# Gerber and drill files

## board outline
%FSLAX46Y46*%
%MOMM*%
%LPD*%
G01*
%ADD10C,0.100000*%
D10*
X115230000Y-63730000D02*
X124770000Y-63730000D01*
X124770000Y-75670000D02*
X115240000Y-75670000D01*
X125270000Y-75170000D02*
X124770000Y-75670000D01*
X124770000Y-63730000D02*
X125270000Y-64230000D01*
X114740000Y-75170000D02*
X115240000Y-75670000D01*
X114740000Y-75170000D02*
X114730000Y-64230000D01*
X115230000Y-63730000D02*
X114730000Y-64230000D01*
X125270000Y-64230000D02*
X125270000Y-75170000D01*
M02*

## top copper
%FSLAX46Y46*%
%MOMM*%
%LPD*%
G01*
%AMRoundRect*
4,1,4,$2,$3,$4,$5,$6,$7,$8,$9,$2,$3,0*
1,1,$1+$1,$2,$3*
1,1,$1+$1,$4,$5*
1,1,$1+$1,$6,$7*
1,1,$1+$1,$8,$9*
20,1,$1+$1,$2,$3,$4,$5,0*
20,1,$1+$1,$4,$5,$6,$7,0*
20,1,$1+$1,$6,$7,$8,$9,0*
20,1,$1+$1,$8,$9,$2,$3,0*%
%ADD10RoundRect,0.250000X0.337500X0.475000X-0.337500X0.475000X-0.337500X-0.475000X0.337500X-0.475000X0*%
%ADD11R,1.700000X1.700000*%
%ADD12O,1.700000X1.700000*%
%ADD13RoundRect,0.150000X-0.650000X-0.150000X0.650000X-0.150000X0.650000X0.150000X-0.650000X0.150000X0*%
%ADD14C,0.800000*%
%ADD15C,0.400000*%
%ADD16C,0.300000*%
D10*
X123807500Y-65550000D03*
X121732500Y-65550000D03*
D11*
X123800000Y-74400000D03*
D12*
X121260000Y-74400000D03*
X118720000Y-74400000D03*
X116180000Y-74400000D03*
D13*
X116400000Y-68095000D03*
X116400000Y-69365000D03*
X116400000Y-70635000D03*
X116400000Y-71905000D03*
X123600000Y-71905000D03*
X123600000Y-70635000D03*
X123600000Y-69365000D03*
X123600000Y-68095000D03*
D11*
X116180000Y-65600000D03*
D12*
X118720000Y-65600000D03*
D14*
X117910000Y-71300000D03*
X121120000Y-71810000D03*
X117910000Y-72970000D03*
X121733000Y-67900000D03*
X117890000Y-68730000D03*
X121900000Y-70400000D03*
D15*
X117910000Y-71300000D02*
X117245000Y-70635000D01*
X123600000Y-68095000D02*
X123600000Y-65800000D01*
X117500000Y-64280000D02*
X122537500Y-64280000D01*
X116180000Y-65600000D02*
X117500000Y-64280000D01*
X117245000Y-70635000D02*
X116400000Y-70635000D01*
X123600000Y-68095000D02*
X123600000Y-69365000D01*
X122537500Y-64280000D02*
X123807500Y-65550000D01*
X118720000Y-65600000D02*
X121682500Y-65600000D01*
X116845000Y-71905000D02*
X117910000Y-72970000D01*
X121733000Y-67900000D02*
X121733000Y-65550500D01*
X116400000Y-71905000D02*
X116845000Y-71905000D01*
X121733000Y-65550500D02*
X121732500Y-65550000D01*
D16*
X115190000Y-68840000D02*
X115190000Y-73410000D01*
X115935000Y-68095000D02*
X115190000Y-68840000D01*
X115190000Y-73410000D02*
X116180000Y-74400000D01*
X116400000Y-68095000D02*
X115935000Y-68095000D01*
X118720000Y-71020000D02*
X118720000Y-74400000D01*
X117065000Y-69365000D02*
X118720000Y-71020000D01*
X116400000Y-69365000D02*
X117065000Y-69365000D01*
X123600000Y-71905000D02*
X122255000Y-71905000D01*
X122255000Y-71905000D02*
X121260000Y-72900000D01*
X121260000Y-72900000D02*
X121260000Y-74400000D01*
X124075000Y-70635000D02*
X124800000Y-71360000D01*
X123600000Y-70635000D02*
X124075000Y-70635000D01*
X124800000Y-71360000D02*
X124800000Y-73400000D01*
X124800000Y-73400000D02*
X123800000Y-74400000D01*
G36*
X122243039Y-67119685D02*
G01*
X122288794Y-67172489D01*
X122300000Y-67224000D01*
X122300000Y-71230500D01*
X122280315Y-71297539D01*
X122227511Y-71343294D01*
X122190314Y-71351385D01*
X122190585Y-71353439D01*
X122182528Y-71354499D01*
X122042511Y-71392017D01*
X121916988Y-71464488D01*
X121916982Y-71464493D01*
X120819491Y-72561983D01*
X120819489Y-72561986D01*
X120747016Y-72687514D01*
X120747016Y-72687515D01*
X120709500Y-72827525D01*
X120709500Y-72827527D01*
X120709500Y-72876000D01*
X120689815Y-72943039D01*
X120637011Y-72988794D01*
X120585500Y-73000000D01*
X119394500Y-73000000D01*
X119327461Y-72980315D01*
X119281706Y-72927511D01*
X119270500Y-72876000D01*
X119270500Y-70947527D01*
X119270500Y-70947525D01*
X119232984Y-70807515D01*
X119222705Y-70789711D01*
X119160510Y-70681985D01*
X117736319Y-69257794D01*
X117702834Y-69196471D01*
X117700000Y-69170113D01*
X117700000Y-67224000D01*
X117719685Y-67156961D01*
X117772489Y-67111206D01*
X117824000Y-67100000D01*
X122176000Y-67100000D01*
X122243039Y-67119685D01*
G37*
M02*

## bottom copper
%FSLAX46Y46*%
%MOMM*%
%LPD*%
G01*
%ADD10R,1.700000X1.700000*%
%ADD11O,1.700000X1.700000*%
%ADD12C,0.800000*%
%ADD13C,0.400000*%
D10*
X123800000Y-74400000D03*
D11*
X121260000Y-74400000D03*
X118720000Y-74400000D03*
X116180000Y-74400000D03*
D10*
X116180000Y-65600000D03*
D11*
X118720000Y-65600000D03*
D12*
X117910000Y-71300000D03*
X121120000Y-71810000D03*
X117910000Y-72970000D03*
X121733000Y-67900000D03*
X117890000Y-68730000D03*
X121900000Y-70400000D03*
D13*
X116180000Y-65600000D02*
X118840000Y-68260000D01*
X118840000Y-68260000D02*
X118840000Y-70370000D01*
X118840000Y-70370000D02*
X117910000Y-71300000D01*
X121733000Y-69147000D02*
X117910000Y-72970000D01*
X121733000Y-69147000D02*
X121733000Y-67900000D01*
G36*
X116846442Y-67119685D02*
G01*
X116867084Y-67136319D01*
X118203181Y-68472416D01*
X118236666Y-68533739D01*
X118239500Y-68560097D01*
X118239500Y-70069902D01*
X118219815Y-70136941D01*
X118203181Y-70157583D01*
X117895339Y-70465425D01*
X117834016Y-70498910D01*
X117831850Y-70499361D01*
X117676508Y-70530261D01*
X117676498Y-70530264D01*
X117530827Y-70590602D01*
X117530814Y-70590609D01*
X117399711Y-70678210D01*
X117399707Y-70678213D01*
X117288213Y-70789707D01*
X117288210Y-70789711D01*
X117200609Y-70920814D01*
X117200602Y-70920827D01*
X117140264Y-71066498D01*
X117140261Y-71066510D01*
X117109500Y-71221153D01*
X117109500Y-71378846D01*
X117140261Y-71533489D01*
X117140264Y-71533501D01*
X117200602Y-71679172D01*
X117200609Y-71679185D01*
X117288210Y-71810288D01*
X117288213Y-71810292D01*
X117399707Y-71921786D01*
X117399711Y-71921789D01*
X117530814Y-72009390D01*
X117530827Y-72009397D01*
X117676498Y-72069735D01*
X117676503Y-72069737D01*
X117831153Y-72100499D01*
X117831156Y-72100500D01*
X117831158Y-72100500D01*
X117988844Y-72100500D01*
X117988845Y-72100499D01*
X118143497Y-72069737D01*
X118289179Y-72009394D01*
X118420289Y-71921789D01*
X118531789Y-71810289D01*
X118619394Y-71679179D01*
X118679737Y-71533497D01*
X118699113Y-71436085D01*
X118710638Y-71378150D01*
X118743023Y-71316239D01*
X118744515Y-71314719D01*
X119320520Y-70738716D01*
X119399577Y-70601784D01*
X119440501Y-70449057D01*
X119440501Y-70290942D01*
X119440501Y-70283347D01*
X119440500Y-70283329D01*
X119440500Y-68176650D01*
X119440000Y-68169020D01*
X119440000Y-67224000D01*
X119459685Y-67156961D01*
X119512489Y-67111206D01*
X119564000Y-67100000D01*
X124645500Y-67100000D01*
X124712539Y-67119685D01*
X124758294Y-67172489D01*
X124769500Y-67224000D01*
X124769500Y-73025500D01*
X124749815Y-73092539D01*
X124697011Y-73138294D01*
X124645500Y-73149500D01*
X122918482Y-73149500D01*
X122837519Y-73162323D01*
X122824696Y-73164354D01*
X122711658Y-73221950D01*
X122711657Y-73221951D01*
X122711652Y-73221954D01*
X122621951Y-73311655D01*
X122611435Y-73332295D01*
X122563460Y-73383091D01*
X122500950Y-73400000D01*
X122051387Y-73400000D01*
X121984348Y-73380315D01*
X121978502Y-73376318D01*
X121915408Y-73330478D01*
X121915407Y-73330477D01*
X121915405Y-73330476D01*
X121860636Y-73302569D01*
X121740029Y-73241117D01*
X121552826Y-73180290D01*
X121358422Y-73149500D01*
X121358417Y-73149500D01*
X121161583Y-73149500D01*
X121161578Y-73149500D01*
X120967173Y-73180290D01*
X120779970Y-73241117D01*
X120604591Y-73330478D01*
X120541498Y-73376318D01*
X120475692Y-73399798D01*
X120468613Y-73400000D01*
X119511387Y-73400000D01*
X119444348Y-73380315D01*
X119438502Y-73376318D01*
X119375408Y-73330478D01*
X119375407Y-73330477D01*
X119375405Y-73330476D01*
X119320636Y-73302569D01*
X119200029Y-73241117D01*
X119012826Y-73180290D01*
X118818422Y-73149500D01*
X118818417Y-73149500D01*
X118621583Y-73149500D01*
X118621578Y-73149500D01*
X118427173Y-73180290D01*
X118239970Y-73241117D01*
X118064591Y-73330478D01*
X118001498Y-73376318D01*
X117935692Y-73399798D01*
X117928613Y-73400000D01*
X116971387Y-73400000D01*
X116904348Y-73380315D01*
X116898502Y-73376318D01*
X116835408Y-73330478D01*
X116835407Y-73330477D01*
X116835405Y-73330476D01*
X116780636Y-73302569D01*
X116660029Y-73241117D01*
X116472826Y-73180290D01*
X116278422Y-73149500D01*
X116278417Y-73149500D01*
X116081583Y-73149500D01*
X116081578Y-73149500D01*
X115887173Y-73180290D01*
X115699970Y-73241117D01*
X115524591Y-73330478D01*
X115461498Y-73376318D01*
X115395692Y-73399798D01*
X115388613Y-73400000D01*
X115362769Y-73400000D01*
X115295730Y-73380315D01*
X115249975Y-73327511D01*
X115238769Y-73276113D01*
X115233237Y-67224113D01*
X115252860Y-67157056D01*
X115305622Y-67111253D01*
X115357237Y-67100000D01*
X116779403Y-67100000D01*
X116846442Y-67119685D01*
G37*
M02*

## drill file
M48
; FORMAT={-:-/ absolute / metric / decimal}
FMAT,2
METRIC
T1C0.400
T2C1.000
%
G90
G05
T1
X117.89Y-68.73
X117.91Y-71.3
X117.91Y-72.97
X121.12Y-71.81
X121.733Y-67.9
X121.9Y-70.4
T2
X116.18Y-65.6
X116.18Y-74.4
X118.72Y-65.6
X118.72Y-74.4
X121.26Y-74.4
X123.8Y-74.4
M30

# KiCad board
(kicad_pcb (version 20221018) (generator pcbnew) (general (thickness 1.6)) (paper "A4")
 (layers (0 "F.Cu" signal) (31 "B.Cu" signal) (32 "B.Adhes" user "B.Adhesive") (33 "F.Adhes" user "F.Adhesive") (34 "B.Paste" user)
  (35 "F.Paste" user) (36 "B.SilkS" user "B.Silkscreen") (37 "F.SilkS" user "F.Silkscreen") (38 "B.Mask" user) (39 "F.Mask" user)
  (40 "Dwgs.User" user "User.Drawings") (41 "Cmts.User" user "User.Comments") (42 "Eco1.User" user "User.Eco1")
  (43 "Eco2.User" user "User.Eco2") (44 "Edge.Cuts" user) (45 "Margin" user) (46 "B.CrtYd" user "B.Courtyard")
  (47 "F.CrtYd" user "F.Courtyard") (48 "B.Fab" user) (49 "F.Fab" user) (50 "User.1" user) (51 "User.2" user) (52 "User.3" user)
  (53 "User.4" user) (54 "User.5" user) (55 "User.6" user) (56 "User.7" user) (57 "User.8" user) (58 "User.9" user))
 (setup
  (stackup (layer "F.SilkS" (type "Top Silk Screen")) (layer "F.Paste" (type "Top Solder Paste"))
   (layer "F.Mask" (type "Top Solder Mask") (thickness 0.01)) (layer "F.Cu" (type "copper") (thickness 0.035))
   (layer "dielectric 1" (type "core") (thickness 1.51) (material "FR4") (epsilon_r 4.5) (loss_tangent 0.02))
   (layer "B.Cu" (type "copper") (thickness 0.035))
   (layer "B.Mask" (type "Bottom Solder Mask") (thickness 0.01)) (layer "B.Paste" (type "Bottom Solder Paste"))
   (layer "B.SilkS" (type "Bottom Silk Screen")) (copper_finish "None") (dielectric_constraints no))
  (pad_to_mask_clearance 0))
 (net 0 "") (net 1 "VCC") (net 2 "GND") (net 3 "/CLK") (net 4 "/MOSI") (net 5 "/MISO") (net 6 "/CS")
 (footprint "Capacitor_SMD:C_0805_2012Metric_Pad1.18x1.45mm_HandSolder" (layer "F.Cu") (at 122.77 65.55 180)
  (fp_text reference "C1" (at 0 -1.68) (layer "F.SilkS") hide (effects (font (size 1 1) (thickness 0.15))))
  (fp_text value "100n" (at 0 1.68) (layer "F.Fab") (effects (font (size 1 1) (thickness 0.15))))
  (pad "1" smd roundrect (at -1.0375 0 180) (size 1.175 1.45) (layers "F.Cu" "F.Paste" "F.Mask") (roundrect_rratio 0.2127659574)
   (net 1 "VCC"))
  (pad "2" smd roundrect (at 1.0375 0 180) (size 1.175 1.45) (layers "F.Cu" "F.Paste" "F.Mask") (roundrect_rratio 0.2127659574)
   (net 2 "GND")))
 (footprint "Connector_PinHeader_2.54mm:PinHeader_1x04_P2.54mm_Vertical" (layer "F.Cu") (at 123.8 74.4 -90)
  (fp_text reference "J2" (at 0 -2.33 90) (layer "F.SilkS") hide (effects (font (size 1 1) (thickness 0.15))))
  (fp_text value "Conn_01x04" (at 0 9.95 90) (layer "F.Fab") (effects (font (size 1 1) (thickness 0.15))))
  (pad "1" thru_hole rect (at 0 0 270) (size 1.7 1.7) (drill 1) (layers "*.Cu" "*.Mask") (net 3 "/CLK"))
  (pad "2" thru_hole oval (at 0 2.54 270) (size 1.7 1.7) (drill 1) (layers "*.Cu" "*.Mask") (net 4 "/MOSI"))
  (pad "3" thru_hole oval (at 0 5.08 270) (size 1.7 1.7) (drill 1) (layers "*.Cu" "*.Mask") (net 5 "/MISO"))
  (pad "4" thru_hole oval (at 0 7.62 270) (size 1.7 1.7) (drill 1) (layers "*.Cu" "*.Mask") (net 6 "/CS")))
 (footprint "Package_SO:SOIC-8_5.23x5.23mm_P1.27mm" (layer "F.Cu") (at 120 70)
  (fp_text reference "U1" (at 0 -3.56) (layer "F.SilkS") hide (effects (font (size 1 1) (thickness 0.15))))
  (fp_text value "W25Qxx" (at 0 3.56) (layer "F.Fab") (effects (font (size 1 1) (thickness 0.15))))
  (pad "1" smd roundrect (at -3.6 -1.905) (size 1.6 0.6) (layers "F.Cu" "F.Paste" "F.Mask") (roundrect_rratio 0.25) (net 6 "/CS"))
  (pad "2" smd roundrect (at -3.6 -0.635) (size 1.6 0.6) (layers "F.Cu" "F.Paste" "F.Mask") (roundrect_rratio 0.25) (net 5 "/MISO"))
  (pad "3" smd roundrect (at -3.6 0.635) (size 1.6 0.6) (layers "F.Cu" "F.Paste" "F.Mask") (roundrect_rratio 0.25) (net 1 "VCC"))
  (pad "4" smd roundrect (at -3.6 1.905) (size 1.6 0.6) (layers "F.Cu" "F.Paste" "F.Mask") (roundrect_rratio 0.25) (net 2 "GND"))
  (pad "5" smd roundrect (at 3.6 1.905) (size 1.6 0.6) (layers "F.Cu" "F.Paste" "F.Mask") (roundrect_rratio 0.25) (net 4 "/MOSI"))
  (pad "6" smd roundrect (at 3.6 0.635) (size 1.6 0.6) (layers "F.Cu" "F.Paste" "F.Mask") (roundrect_rratio 0.25) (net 3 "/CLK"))
  (pad "7" smd roundrect (at 3.6 -0.635) (size 1.6 0.6) (layers "F.Cu" "F.Paste" "F.Mask") (roundrect_rratio 0.25) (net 1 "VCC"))
  (pad "8" smd roundrect (at 3.6 -1.905) (size 1.6 0.6) (layers "F.Cu" "F.Paste" "F.Mask") (roundrect_rratio 0.25) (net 1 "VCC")))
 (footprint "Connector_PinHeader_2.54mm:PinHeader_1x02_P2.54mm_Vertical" (layer "F.Cu") (at 116.18 65.6 90)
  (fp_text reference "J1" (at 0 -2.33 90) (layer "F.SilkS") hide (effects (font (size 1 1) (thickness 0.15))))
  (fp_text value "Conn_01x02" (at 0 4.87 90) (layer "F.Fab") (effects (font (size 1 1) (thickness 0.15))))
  (pad "1" thru_hole rect (at 0 0 90) (size 1.7 1.7) (drill 1) (layers "*.Cu" "*.Mask") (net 1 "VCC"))
  (pad "2" thru_hole oval (at 0 2.54 90) (size 1.7 1.7) (drill 1) (layers "*.Cu" "*.Mask") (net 2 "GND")))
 (gr_line (start 115.23 63.73) (end 124.77 63.73) (stroke (width 0.1) (type default)) (layer "Edge.Cuts"))
 (gr_line (start 124.77 75.67) (end 115.24 75.67) (stroke (width 0.1) (type default)) (layer "Edge.Cuts"))
 (gr_line (start 125.27 75.17) (end 124.77 75.67) (stroke (width 0.1) (type default)) (layer "Edge.Cuts"))
 (gr_line (start 124.77 63.73) (end 125.27 64.23) (stroke (width 0.1) (type default)) (layer "Edge.Cuts"))
 (gr_line (start 114.74 75.17) (end 115.24 75.67) (stroke (width 0.1) (type default)) (layer "Edge.Cuts"))
 (gr_line (start 114.74 75.17) (end 114.73 64.23) (stroke (width 0.1) (type default)) (layer "Edge.Cuts"))
 (gr_line (start 115.23 63.73) (end 114.73 64.23) (stroke (width 0.1) (type default)) (layer "Edge.Cuts"))
 (gr_line (start 125.27 64.23) (end 125.27 75.17) (stroke (width 0.1) (type default)) (layer "Edge.Cuts"))
 (segment (start 117.91 71.3) (end 117.245 70.635) (width 0.4) (layer "F.Cu") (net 1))
 (segment (start 123.6 68.095) (end 123.6 65.8) (width 0.4) (layer "F.Cu") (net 1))
 (segment (start 117.5 64.28) (end 122.5375 64.28) (width 0.4) (layer "F.Cu") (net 1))
 (segment (start 116.18 65.6) (end 117.5 64.28) (width 0.4) (layer "F.Cu") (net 1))
 (segment (start 117.245 70.635) (end 116.4 70.635) (width 0.4) (layer "F.Cu") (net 1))
 (segment (start 123.6 68.095) (end 123.6 69.365) (width 0.4) (layer "F.Cu") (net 1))
 (segment (start 122.5375 64.28) (end 123.8075 65.55) (width 0.4) (layer "F.Cu") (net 1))
 (via (at 117.91 71.3) (size 0.8) (drill 0.4) (layers "F.Cu" "B.Cu") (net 1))
 (segment (start 116.18 65.6) (end 118.84 68.26) (width 0.4) (layer "B.Cu") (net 1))
 (segment (start 118.84 68.26) (end 118.84 70.37) (width 0.4) (layer "B.Cu") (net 1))
 (segment (start 118.84 70.37) (end 117.91 71.3) (width 0.4) (layer "B.Cu") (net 1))
 (segment (start 118.72 65.6) (end 121.6825 65.6) (width 0.4) (layer "F.Cu") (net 2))
 (segment (start 116.845 71.905) (end 117.91 72.97) (width 0.4) (layer "F.Cu") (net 2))
 (segment (start 121.733 67.9) (end 121.733 65.5505) (width 0.4) (layer "F.Cu") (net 2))
 (segment (start 116.4 71.905) (end 116.845 71.905) (width 0.4) (layer "F.Cu") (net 2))
 (segment (start 121.733 65.5505) (end 121.7325 65.55) (width 0.4) (layer "F.Cu") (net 2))
 (via (at 121.12 71.81) (size 0.8) (drill 0.4) (layers "F.Cu" "B.Cu") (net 2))
 (via (at 117.91 72.97) (size 0.8) (drill 0.4) (layers "F.Cu" "B.Cu") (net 2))
 (via (at 121.733 67.9) (size 0.8) (drill 0.4) (layers "F.Cu" "B.Cu") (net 2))
 (via (at 117.89 68.73) (size 0.8) (drill 0.4) (layers "F.Cu" "B.Cu") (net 2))
 (via (at 121.9 70.4) (size 0.8) (drill 0.4) (layers "F.Cu" "B.Cu") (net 2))
 (segment (start 121.733 69.147) (end 117.91 72.97) (width 0.4) (layer "B.Cu") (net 2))
 (segment (start 121.733 69.147) (end 121.733 67.9) (width 0.4) (layer "B.Cu") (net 2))
 (segment (start 115.19 68.84) (end 115.19 73.41) (width 0.3) (layer "F.Cu") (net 6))
 (segment (start 115.935 68.095) (end 115.19 68.84) (width 0.3) (layer "F.Cu") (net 6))
 (segment (start 115.19 73.41) (end 116.18 74.4) (width 0.3) (layer "F.Cu") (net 6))
 (segment (start 116.4 68.095) (end 115.935 68.095) (width 0.3) (layer "F.Cu") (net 6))
 (segment (start 118.72 71.02) (end 118.72 74.4) (width 0.3) (layer "F.Cu") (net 5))
 (segment (start 117.065 69.365) (end 118.72 71.02) (width 0.3) (layer "F.Cu") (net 5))
 (segment (start 116.4 69.365) (end 117.065 69.365) (width 0.3) (layer "F.Cu") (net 5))
 (segment (start 123.6 71.905) (end 122.255 71.905) (width 0.3) (layer "F.Cu") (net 4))
 (segment (start 122.255 71.905) (end 121.26 72.9) (width 0.3) (layer "F.Cu") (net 4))
 (segment (start 121.26 72.9) (end 121.26 74.4) (width 0.3) (layer "F.Cu") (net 4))
 (segment (start 124.075 70.635) (end 124.8 71.36) (width 0.3) (layer "F.Cu") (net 3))
 (segment (start 123.6 70.635) (end 124.075 70.635) (width 0.3) (layer "F.Cu") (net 3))
 (segment (start 124.8 71.36) (end 124.8 73.4) (width 0.3) (layer "F.Cu") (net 3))
 (segment (start 124.8 73.4) (end 123.8 74.4) (width 0.3) (layer "F.Cu") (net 3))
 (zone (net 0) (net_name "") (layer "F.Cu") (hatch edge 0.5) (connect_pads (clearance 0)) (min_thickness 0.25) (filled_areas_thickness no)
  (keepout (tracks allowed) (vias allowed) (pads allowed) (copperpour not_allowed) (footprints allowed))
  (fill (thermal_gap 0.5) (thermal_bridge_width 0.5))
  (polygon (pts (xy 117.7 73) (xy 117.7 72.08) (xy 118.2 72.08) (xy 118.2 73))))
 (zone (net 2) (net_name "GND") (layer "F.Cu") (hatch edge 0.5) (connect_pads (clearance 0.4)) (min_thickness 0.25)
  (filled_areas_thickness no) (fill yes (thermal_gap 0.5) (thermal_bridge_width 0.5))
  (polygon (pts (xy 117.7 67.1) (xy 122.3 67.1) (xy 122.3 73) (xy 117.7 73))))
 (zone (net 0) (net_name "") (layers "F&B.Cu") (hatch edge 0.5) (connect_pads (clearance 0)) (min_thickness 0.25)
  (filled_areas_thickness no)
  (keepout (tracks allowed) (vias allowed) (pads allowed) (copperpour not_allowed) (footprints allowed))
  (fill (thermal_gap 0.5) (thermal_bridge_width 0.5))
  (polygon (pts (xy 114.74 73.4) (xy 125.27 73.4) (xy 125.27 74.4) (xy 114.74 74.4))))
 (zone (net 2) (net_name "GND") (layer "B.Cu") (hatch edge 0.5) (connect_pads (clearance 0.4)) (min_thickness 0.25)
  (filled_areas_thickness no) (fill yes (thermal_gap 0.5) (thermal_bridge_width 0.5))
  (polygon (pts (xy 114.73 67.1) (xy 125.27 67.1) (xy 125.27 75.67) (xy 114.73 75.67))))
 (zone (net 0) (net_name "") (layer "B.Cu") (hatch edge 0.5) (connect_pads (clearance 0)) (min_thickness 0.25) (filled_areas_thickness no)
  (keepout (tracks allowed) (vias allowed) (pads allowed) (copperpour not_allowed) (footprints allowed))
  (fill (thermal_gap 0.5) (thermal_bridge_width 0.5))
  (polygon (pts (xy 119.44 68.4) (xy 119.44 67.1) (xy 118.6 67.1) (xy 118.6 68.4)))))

